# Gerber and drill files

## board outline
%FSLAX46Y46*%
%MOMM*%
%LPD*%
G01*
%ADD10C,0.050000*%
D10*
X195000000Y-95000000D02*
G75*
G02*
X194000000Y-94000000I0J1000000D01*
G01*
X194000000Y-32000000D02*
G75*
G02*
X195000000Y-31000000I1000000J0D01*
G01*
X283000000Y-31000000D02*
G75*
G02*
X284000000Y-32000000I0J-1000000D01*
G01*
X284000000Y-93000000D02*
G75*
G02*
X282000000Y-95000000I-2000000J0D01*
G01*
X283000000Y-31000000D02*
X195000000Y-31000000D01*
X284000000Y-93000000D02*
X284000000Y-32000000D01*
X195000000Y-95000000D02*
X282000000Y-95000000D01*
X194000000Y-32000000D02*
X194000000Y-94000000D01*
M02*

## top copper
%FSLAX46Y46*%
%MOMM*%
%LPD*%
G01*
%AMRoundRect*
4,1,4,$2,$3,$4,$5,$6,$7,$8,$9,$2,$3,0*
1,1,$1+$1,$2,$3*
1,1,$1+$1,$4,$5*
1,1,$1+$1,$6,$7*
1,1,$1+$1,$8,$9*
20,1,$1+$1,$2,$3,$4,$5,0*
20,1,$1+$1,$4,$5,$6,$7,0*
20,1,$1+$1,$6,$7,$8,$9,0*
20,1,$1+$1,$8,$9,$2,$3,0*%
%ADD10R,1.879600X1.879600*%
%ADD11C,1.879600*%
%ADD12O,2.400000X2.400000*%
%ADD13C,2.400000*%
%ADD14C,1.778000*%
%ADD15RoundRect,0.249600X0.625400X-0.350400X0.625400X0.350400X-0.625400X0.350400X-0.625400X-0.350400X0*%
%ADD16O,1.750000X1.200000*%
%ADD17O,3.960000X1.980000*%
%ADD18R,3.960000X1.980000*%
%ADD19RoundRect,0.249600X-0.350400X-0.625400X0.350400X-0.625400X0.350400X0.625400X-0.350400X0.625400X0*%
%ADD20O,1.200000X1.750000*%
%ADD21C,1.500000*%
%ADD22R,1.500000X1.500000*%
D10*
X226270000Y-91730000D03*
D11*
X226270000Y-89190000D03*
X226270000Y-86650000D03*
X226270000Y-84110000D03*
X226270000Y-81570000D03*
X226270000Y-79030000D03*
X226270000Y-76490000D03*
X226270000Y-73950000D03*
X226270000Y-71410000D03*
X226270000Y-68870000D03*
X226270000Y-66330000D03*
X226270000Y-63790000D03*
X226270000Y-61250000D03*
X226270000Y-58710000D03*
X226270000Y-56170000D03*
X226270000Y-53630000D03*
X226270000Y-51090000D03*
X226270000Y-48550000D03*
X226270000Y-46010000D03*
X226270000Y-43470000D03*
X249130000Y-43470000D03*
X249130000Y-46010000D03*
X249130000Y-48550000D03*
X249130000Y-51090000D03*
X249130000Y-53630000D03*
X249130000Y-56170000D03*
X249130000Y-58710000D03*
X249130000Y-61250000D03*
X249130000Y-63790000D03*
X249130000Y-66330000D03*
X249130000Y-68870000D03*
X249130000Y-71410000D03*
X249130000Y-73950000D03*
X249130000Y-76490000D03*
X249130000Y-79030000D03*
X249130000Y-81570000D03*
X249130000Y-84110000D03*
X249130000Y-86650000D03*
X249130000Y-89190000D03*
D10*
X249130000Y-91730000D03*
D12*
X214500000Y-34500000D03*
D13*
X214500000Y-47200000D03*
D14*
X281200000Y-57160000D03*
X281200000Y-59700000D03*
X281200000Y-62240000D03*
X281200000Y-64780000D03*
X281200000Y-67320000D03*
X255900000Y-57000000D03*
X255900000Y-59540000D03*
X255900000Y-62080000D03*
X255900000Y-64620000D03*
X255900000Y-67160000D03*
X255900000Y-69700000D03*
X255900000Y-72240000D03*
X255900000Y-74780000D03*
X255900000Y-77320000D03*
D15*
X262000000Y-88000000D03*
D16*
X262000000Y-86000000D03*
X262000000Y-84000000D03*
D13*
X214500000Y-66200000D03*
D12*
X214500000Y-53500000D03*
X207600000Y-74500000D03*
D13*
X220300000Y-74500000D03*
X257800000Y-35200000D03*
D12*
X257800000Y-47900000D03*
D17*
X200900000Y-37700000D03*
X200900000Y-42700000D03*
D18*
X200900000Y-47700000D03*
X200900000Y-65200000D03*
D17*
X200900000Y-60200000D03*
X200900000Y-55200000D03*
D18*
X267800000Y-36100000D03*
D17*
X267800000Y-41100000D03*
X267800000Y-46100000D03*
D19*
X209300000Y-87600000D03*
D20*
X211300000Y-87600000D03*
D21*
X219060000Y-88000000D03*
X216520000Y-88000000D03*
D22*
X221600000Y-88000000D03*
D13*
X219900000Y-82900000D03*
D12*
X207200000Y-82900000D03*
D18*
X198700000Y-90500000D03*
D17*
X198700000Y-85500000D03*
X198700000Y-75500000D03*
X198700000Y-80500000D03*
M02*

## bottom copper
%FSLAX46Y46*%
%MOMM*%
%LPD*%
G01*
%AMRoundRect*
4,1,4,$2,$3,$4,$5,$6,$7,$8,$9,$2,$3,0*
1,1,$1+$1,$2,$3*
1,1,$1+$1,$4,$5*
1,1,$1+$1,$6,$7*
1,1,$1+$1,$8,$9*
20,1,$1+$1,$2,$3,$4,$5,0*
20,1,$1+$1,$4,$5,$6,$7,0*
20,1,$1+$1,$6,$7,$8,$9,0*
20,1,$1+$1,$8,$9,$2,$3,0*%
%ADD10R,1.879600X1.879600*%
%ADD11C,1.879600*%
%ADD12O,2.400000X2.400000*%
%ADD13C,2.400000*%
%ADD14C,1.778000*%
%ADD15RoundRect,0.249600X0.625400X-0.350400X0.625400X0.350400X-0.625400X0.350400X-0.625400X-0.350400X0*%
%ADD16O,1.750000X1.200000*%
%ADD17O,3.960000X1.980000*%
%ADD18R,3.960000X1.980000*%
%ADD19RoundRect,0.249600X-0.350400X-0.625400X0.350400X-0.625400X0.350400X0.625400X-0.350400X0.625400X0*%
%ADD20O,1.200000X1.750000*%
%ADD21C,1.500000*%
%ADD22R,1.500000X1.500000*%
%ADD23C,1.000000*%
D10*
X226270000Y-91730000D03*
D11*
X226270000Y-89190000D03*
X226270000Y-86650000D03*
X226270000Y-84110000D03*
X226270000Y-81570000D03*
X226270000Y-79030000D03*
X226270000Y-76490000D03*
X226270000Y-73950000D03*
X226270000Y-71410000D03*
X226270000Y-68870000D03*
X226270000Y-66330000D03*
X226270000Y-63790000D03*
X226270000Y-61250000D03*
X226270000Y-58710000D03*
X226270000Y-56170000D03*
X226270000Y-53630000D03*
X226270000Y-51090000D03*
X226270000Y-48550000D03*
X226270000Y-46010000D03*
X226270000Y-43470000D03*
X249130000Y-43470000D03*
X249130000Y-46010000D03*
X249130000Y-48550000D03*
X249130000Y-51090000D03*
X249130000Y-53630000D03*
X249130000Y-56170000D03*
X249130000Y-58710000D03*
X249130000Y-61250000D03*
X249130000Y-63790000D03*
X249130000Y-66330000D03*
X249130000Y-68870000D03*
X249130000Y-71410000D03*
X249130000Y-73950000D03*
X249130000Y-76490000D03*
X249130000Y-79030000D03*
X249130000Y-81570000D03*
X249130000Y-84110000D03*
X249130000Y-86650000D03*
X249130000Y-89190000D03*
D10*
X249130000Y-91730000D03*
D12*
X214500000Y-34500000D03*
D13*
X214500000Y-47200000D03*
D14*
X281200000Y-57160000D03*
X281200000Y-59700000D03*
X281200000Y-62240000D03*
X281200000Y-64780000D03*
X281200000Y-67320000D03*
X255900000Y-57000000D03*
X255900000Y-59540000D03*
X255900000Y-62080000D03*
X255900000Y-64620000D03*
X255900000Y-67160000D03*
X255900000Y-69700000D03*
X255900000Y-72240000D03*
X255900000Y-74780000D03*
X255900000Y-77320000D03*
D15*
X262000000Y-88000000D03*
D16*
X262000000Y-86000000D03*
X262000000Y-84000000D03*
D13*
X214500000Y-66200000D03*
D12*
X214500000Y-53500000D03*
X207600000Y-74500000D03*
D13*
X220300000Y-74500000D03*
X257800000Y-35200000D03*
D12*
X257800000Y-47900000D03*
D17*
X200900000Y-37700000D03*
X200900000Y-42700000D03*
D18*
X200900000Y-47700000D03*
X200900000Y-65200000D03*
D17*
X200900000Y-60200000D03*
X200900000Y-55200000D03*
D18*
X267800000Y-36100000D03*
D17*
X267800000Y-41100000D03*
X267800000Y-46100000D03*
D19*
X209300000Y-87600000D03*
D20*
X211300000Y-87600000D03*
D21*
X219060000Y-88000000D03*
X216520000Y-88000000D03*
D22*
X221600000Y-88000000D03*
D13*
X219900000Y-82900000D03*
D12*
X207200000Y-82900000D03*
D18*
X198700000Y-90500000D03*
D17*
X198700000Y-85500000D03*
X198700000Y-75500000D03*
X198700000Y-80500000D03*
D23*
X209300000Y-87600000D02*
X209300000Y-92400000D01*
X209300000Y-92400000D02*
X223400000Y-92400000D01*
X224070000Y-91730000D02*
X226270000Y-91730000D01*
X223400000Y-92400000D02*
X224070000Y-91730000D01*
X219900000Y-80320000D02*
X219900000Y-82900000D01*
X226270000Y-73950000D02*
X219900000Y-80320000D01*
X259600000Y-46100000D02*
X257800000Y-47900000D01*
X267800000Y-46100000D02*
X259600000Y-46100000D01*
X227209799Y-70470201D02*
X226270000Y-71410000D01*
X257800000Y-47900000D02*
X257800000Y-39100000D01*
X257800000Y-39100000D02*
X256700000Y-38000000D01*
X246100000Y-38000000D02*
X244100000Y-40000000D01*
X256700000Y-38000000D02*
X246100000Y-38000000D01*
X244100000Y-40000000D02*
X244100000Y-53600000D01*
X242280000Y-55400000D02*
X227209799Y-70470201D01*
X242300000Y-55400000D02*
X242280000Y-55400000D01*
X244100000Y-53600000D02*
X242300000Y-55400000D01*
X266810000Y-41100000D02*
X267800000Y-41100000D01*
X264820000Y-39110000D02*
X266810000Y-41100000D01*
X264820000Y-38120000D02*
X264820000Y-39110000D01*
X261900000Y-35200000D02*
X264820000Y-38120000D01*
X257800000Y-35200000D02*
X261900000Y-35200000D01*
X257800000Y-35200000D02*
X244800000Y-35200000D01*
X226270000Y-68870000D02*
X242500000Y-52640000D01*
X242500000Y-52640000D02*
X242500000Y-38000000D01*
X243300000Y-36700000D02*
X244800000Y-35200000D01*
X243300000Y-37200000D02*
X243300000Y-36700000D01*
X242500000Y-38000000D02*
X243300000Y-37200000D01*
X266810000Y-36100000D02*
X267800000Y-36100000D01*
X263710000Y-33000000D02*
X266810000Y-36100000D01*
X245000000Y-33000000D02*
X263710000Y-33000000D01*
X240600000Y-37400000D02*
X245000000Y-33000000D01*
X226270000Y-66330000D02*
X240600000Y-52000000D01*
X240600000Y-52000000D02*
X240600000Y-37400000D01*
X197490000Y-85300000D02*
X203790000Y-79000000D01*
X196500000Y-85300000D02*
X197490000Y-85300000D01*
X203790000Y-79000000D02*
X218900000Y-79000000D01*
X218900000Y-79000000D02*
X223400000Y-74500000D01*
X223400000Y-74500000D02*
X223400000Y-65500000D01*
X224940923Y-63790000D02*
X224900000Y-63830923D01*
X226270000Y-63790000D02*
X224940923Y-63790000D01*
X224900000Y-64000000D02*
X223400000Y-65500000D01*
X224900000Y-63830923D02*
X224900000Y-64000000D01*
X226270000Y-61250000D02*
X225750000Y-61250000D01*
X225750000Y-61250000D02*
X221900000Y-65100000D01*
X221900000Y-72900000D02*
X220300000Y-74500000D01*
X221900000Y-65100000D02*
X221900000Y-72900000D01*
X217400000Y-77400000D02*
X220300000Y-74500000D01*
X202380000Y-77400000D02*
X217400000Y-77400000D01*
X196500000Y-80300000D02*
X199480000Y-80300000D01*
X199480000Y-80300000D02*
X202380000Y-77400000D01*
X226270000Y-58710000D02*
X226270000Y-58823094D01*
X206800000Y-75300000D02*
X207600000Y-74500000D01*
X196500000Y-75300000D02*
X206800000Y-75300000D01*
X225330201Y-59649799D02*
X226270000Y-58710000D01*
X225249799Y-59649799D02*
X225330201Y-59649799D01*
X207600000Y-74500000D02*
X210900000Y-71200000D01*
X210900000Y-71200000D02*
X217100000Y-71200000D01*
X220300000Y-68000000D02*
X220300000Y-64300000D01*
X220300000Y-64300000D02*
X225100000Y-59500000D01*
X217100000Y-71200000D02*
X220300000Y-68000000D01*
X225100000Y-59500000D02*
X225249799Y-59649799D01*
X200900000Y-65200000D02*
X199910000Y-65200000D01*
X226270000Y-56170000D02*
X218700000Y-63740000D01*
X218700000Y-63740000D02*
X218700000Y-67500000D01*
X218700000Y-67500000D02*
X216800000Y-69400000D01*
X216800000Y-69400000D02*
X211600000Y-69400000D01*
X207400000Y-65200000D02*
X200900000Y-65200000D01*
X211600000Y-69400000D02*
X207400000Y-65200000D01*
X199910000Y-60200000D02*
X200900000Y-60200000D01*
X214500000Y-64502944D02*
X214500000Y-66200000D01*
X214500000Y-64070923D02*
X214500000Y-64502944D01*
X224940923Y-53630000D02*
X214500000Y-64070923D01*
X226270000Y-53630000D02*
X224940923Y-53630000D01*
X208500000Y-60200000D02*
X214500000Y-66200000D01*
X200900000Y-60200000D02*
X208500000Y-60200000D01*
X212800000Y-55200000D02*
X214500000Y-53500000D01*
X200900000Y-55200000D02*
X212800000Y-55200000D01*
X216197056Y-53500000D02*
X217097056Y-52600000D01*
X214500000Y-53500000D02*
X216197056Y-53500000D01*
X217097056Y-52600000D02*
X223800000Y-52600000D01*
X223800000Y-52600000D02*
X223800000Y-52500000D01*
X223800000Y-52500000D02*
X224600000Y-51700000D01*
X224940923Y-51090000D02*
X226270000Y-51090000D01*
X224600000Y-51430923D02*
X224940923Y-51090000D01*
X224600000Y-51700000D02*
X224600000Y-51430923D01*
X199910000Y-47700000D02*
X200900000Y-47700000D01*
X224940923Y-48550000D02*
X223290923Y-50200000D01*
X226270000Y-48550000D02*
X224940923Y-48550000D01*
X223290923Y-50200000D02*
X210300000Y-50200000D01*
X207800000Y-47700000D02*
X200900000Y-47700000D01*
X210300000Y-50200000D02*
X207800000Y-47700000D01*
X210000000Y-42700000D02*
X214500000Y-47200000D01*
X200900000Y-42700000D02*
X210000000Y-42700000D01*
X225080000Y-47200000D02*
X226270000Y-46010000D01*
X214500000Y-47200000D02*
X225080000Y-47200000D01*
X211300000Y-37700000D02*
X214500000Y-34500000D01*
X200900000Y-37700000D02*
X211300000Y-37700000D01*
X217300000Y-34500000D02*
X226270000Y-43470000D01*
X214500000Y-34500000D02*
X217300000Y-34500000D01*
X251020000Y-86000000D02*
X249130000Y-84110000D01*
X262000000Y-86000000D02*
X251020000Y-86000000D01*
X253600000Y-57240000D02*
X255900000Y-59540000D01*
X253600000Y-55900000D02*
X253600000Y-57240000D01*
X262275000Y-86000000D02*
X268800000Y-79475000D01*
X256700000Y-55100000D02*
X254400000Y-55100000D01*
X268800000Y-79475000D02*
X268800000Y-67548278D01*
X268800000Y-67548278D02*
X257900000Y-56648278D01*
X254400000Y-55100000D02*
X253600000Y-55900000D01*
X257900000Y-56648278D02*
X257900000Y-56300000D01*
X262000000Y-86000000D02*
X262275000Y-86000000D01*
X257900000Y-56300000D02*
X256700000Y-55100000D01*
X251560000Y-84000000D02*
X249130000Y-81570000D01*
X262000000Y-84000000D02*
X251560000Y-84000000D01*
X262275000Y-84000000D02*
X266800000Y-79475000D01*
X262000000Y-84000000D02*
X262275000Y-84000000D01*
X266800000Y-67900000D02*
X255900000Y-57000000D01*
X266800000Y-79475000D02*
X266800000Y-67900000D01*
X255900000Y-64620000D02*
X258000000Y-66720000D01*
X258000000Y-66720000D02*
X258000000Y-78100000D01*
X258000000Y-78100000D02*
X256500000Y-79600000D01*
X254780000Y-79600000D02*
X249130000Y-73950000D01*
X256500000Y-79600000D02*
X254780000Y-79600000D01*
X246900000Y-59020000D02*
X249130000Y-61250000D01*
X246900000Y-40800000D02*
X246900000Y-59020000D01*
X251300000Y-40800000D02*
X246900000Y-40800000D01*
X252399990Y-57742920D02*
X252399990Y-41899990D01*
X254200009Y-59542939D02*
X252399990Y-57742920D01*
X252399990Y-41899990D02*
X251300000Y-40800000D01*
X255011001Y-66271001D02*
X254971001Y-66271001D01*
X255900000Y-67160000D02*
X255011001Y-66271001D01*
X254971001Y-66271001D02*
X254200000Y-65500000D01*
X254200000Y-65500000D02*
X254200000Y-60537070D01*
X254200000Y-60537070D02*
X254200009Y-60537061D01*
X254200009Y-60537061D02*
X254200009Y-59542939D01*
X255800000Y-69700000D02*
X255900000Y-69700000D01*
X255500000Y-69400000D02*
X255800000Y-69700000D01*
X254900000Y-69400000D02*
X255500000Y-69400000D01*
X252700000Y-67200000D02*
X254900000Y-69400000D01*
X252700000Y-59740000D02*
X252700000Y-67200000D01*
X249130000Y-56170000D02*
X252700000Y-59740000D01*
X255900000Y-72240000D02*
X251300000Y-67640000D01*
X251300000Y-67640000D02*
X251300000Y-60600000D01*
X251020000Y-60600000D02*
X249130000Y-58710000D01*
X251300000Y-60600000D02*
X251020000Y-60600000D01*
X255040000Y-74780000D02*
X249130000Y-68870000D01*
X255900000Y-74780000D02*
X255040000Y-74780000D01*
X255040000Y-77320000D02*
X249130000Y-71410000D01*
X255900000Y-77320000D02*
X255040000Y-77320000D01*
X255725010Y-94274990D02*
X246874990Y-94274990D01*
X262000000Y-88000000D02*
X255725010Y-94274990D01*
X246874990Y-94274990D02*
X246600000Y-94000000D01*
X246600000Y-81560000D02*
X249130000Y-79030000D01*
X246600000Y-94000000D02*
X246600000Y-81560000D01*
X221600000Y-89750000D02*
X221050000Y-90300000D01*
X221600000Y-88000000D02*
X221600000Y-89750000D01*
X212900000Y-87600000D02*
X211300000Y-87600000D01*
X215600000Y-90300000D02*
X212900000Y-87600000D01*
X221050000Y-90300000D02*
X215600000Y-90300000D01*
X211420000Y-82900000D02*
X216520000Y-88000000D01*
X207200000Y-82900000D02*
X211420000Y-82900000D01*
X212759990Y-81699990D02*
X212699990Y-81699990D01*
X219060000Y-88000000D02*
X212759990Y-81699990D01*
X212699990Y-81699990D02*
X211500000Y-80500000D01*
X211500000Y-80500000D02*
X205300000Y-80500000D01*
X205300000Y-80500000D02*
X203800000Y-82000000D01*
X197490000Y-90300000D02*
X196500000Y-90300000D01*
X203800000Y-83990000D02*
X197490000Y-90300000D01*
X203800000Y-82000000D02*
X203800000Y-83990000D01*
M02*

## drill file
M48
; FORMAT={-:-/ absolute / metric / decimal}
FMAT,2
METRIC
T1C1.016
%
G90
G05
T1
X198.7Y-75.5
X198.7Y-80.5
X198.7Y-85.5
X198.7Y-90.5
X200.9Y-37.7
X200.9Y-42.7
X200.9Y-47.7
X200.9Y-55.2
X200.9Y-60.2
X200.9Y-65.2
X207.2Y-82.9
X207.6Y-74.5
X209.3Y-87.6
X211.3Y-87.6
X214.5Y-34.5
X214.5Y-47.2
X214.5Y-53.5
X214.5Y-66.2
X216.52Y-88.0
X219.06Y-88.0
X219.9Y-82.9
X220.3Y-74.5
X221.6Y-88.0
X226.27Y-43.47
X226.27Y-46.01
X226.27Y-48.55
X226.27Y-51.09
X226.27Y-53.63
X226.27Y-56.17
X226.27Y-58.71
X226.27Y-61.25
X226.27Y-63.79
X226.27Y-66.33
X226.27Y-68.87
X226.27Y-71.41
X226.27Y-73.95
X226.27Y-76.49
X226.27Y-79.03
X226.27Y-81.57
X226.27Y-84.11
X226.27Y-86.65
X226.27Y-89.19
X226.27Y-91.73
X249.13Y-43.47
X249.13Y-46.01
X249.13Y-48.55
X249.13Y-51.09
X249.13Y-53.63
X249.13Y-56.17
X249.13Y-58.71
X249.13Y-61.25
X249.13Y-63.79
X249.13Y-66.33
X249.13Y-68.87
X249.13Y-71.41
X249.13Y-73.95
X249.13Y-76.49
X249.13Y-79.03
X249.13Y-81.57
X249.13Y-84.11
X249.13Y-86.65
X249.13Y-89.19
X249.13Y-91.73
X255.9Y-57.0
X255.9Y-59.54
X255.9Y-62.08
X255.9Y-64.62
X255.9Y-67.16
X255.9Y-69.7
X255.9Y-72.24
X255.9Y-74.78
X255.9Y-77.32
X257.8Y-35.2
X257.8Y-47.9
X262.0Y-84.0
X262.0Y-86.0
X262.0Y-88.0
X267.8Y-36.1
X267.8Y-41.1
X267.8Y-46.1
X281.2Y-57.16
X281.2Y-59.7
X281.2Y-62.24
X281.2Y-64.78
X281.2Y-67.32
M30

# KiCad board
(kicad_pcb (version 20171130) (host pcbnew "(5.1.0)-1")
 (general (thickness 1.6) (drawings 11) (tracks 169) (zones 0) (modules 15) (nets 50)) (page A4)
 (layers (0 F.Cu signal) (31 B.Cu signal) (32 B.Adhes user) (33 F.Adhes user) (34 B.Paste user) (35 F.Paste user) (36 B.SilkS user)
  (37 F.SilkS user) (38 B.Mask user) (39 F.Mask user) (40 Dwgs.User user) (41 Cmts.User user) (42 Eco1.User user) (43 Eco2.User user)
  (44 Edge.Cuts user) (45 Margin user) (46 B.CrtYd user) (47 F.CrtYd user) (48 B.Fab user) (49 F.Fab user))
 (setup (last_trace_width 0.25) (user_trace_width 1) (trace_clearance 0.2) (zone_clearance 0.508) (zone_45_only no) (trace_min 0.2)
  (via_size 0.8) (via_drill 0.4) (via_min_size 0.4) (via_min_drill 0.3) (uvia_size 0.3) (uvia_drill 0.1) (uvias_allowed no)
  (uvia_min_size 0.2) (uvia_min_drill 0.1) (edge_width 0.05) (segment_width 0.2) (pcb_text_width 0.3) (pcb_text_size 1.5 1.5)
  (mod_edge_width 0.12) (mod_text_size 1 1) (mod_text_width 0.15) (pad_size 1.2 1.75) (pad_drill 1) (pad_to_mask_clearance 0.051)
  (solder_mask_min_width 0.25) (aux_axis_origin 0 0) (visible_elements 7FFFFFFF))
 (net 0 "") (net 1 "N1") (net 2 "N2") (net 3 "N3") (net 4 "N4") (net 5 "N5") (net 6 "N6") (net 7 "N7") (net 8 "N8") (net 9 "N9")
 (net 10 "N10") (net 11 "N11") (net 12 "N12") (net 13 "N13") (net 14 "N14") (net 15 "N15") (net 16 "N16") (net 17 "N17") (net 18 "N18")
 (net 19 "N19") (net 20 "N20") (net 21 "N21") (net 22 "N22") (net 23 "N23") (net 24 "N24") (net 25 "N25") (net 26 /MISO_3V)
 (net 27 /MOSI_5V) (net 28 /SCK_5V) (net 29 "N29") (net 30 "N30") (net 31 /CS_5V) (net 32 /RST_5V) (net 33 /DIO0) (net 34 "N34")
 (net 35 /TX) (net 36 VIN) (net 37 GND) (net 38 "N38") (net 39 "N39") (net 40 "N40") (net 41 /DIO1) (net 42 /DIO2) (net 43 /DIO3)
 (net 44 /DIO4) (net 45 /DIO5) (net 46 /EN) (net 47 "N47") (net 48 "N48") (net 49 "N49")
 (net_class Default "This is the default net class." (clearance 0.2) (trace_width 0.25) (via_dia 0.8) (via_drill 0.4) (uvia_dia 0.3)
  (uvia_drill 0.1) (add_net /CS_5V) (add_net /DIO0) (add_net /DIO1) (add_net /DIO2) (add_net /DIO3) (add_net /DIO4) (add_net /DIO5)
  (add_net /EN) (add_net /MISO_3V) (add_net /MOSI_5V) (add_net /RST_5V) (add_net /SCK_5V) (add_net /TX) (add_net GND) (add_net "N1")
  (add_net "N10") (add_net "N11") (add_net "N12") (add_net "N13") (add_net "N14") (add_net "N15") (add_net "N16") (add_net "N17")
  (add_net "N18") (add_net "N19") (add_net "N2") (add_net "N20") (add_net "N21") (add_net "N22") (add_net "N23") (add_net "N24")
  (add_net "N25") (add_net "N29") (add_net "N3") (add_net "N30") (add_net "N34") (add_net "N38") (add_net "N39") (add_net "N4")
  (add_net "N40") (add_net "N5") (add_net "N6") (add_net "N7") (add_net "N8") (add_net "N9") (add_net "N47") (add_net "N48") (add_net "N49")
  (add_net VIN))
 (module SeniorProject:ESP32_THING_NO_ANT (layer F.Cu) (at 225 93)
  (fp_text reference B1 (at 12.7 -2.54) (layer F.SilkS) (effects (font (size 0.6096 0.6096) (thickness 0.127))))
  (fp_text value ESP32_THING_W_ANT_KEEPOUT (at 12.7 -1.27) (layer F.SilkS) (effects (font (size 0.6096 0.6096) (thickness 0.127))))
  (pad 1 thru_hole rect (at 1.27 -1.27) (size 1.8796 1.8796) (drill 1.016) (layers *.Cu *.Mask) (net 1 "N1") (solder_mask_margin 0.1016))
  (pad 2 thru_hole circle (at 1.27 -3.81) (size 1.8796 1.8796) (drill 1.016) (layers *.Cu *.Mask) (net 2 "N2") (solder_mask_margin 0.1016))
  (pad 3 thru_hole circle (at 1.27 -6.35) (size 1.8796 1.8796) (drill 1.016) (layers *.Cu *.Mask) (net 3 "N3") (solder_mask_margin 0.1016))
  (pad 4 thru_hole circle (at 1.27 -8.89) (size 1.8796 1.8796) (drill 1.016) (layers *.Cu *.Mask) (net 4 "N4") (solder_mask_margin 0.1016))
  (pad 5 thru_hole circle (at 1.27 -11.43) (size 1.8796 1.8796) (drill 1.016) (layers *.Cu *.Mask) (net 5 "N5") (solder_mask_margin 0.1016))
  (pad 6 thru_hole circle (at 1.27 -13.97) (size 1.8796 1.8796) (drill 1.016) (layers *.Cu *.Mask) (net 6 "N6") (solder_mask_margin 0.1016))
  (pad 7 thru_hole circle (at 1.27 -16.51) (size 1.8796 1.8796) (drill 1.016) (layers *.Cu *.Mask) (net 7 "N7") (solder_mask_margin 0.1016))
  (pad 8 thru_hole circle (at 1.27 -19.05) (size 1.8796 1.8796) (drill 1.016) (layers *.Cu *.Mask) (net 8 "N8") (solder_mask_margin 0.1016))
  (pad 9 thru_hole circle (at 1.27 -21.59) (size 1.8796 1.8796) (drill 1.016) (layers *.Cu *.Mask) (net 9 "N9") (solder_mask_margin 0.1016))
  (pad 10 thru_hole circle (at 1.27 -24.13) (size 1.8796 1.8796) (drill 1.016) (layers *.Cu *.Mask) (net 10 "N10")
   (solder_mask_margin 0.1016))
  (pad 11 thru_hole circle (at 1.27 -26.67) (size 1.8796 1.8796) (drill 1.016) (layers *.Cu *.Mask) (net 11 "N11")
   (solder_mask_margin 0.1016))
  (pad 12 thru_hole circle (at 1.27 -29.21) (size 1.8796 1.8796) (drill 1.016) (layers *.Cu *.Mask) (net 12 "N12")
   (solder_mask_margin 0.1016))
  (pad 13 thru_hole circle (at 1.27 -31.75) (size 1.8796 1.8796) (drill 1.016) (layers *.Cu *.Mask) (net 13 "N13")
   (solder_mask_margin 0.1016))
  (pad 14 thru_hole circle (at 1.27 -34.29) (size 1.8796 1.8796) (drill 1.016) (layers *.Cu *.Mask) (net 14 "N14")
   (solder_mask_margin 0.1016))
  (pad 15 thru_hole circle (at 1.27 -36.83) (size 1.8796 1.8796) (drill 1.016) (layers *.Cu *.Mask) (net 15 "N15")
   (solder_mask_margin 0.1016))
  (pad 16 thru_hole circle (at 1.27 -39.37) (size 1.8796 1.8796) (drill 1.016) (layers *.Cu *.Mask) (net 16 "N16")
   (solder_mask_margin 0.1016))
  (pad 17 thru_hole circle (at 1.27 -41.91) (size 1.8796 1.8796) (drill 1.016) (layers *.Cu *.Mask) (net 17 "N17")
   (solder_mask_margin 0.1016))
  (pad 18 thru_hole circle (at 1.27 -44.45) (size 1.8796 1.8796) (drill 1.016) (layers *.Cu *.Mask) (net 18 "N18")
   (solder_mask_margin 0.1016))
  (pad 19 thru_hole circle (at 1.27 -46.99) (size 1.8796 1.8796) (drill 1.016) (layers *.Cu *.Mask) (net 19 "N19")
   (solder_mask_margin 0.1016))
  (pad 20 thru_hole circle (at 1.27 -49.53) (size 1.8796 1.8796) (drill 1.016) (layers *.Cu *.Mask) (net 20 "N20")
   (solder_mask_margin 0.1016))
  (pad 21 thru_hole circle (at 24.13 -49.53) (size 1.8796 1.8796) (drill 1.016) (layers *.Cu *.Mask) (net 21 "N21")
   (solder_mask_margin 0.1016))
  (pad 22 thru_hole circle (at 24.13 -46.99) (size 1.8796 1.8796) (drill 1.016) (layers *.Cu *.Mask) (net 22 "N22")
   (solder_mask_margin 0.1016))
  (pad 23 thru_hole circle (at 24.13 -44.45) (size 1.8796 1.8796) (drill 1.016) (layers *.Cu *.Mask) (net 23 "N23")
   (solder_mask_margin 0.1016))
  (pad 24 thru_hole circle (at 24.13 -41.91) (size 1.8796 1.8796) (drill 1.016) (layers *.Cu *.Mask) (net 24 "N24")
   (solder_mask_margin 0.1016))
  (pad 25 thru_hole circle (at 24.13 -39.37) (size 1.8796 1.8796) (drill 1.016) (layers *.Cu *.Mask) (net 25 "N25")
   (solder_mask_margin 0.1016))
  (pad 26 thru_hole circle (at 24.13 -36.83) (size 1.8796 1.8796) (drill 1.016) (layers *.Cu *.Mask) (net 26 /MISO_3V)
   (solder_mask_margin 0.1016))
  (pad 27 thru_hole circle (at 24.13 -34.29) (size 1.8796 1.8796) (drill 1.016) (layers *.Cu *.Mask) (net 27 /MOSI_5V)
   (solder_mask_margin 0.1016))
  (pad 28 thru_hole circle (at 24.13 -31.75) (size 1.8796 1.8796) (drill 1.016) (layers *.Cu *.Mask) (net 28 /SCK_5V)
   (solder_mask_margin 0.1016))
  (pad 29 thru_hole circle (at 24.13 -29.21) (size 1.8796 1.8796) (drill 1.016) (layers *.Cu *.Mask) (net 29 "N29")
   (solder_mask_margin 0.1016))
  (pad 30 thru_hole circle (at 24.13 -26.67) (size 1.8796 1.8796) (drill 1.016) (layers *.Cu *.Mask) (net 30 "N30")
   (solder_mask_margin 0.1016))
  (pad 31 thru_hole circle (at 24.13 -24.13) (size 1.8796 1.8796) (drill 1.016) (layers *.Cu *.Mask) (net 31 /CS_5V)
   (solder_mask_margin 0.1016))
  (pad 32 thru_hole circle (at 24.13 -21.59) (size 1.8796 1.8796) (drill 1.016) (layers *.Cu *.Mask) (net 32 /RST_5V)
   (solder_mask_margin 0.1016))
  (pad 33 thru_hole circle (at 24.13 -19.05) (size 1.8796 1.8796) (drill 1.016) (layers *.Cu *.Mask) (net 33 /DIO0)
   (solder_mask_margin 0.1016))
  (pad 34 thru_hole circle (at 24.13 -16.51) (size 1.8796 1.8796) (drill 1.016) (layers *.Cu *.Mask) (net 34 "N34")
   (solder_mask_margin 0.1016))
  (pad 35 thru_hole circle (at 24.13 -13.97) (size 1.8796 1.8796) (drill 1.016) (layers *.Cu *.Mask) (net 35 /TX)
   (solder_mask_margin 0.1016))
  (pad 36 thru_hole circle (at 24.13 -11.43) (size 1.8796 1.8796) (drill 1.016) (layers *.Cu *.Mask) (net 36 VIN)
   (solder_mask_margin 0.1016))
  (pad 37 thru_hole circle (at 24.13 -8.89) (size 1.8796 1.8796) (drill 1.016) (layers *.Cu *.Mask) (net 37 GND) (solder_mask_margin 0.1016))
  (pad 38 thru_hole circle (at 24.13 -6.35) (size 1.8796 1.8796) (drill 1.016) (layers *.Cu *.Mask) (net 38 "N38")
   (solder_mask_margin 0.1016))
  (pad 39 thru_hole circle (at 24.13 -3.81) (size 1.8796 1.8796) (drill 1.016) (layers *.Cu *.Mask) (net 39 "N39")
   (solder_mask_margin 0.1016))
  (pad 40 thru_hole rect (at 24.13 -1.27) (size 1.8796 1.8796) (drill 1.016) (layers *.Cu *.Mask) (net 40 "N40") (solder_mask_margin 0.1016)))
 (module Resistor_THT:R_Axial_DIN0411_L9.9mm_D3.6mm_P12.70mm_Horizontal (layer F.Cu) (at 214.5 47.2 90)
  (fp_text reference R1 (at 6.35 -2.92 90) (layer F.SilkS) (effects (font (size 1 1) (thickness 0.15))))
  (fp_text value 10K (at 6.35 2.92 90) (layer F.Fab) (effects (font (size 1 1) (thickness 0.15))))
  (pad 2 thru_hole oval (at 12.7 0 90) (size 2.4 2.4) (drill 1.016) (layers *.Cu *.Mask) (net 20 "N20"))
  (pad 1 thru_hole circle (at 0 0 90) (size 2.4 2.4) (drill 1.016) (layers *.Cu *.Mask) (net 19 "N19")))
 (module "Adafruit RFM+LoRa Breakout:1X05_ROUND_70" (layer F.Cu) (at 281.2 62.24 270)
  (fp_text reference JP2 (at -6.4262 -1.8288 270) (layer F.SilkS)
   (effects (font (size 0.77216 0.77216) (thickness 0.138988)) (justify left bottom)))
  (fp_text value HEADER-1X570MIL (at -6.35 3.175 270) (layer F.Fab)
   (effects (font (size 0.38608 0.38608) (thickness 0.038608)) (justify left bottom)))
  (pad 1 thru_hole circle (at -5.08 0) (size 1.778 1.778) (drill 1.016) (layers *.Cu *.Mask) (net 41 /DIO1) (solder_mask_margin 0.0508))
  (pad 2 thru_hole circle (at -2.54 0) (size 1.778 1.778) (drill 1.016) (layers *.Cu *.Mask) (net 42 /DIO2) (solder_mask_margin 0.0508))
  (pad 3 thru_hole circle (at 0 0) (size 1.778 1.778) (drill 1.016) (layers *.Cu *.Mask) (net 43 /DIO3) (solder_mask_margin 0.0508))
  (pad 4 thru_hole circle (at 2.54 0) (size 1.778 1.778) (drill 1.016) (layers *.Cu *.Mask) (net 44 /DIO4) (solder_mask_margin 0.0508))
  (pad 5 thru_hole circle (at 5.08 0) (size 1.778 1.778) (drill 1.016) (layers *.Cu *.Mask) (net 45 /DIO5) (solder_mask_margin 0.0508)))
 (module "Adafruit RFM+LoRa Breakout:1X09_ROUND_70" (layer F.Cu) (at 255.9 67.16 270)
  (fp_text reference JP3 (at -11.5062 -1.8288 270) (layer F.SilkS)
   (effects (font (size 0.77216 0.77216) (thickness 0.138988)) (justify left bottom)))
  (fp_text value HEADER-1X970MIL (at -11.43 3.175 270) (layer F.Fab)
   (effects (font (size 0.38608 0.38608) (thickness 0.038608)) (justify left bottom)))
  (pad 1 thru_hole circle (at -10.16 0) (size 1.778 1.778) (drill 1.016) (layers *.Cu *.Mask) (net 36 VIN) (solder_mask_margin 0.0508))
  (pad 2 thru_hole circle (at -7.62 0) (size 1.778 1.778) (drill 1.016) (layers *.Cu *.Mask) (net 37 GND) (solder_mask_margin 0.0508))
  (pad 3 thru_hole circle (at -5.08 0) (size 1.778 1.778) (drill 1.016) (layers *.Cu *.Mask) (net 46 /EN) (solder_mask_margin 0.0508))
  (pad 4 thru_hole circle (at -2.54 0) (size 1.778 1.778) (drill 1.016) (layers *.Cu *.Mask) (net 33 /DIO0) (solder_mask_margin 0.0508))
  (pad 5 thru_hole circle (at 0 0) (size 1.778 1.778) (drill 1.016) (layers *.Cu *.Mask) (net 28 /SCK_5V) (solder_mask_margin 0.0508))
  (pad 6 thru_hole circle (at 2.54 0) (size 1.778 1.778) (drill 1.016) (layers *.Cu *.Mask) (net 26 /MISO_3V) (solder_mask_margin 0.0508))
  (pad 7 thru_hole circle (at 5.08 0) (size 1.778 1.778) (drill 1.016) (layers *.Cu *.Mask) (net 27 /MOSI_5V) (solder_mask_margin 0.0508))
  (pad 8 thru_hole circle (at 7.62 0) (size 1.778 1.778) (drill 1.016) (layers *.Cu *.Mask) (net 31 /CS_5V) (solder_mask_margin 0.0508))
  (pad 9 thru_hole circle (at 10.16 0) (size 1.778 1.778) (drill 1.016) (layers *.Cu *.Mask) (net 32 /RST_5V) (solder_mask_margin 0.0508)))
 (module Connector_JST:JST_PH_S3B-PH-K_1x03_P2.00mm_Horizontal (layer F.Cu) (at 262 88 90)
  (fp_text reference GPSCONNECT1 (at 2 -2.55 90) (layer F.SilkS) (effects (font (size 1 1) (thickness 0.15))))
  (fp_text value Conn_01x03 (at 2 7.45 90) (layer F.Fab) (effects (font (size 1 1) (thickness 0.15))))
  (pad 1 thru_hole roundrect (at 0 0 90) (size 1.2 1.75) (drill 1.016) (layers *.Cu *.Mask) (roundrect_rratio 0.208) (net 35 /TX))
  (pad 2 thru_hole oval (at 2 0 90) (size 1.2 1.75) (drill 1.016) (layers *.Cu *.Mask) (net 37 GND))
  (pad 3 thru_hole oval (at 4 0 90) (size 1.2 1.75) (drill 1.016) (layers *.Cu *.Mask) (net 36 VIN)))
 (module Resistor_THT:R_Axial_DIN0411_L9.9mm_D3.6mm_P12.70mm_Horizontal (layer F.Cu) (at 214.5 66.2 90)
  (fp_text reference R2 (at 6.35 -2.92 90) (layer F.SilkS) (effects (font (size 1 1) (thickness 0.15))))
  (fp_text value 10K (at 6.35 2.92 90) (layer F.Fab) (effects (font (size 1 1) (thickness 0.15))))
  (pad 1 thru_hole circle (at 0 0 90) (size 2.4 2.4) (drill 1.016) (layers *.Cu *.Mask) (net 16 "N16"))
  (pad 2 thru_hole oval (at 12.7 0 90) (size 2.4 2.4) (drill 1.016) (layers *.Cu *.Mask) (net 17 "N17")))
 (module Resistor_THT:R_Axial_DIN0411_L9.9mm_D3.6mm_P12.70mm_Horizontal (layer F.Cu) (at 220.3 74.5 180)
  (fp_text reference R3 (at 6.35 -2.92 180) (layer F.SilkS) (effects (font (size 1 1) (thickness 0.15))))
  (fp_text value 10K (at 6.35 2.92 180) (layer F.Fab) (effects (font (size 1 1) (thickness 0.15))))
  (pad 2 thru_hole oval (at 12.7 0 180) (size 2.4 2.4) (drill 1.016) (layers *.Cu *.Mask) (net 14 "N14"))
  (pad 1 thru_hole circle (at 0 0 180) (size 2.4 2.4) (drill 1.016) (layers *.Cu *.Mask) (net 13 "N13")))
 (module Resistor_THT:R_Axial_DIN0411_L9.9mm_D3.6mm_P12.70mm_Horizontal (layer F.Cu) (at 257.8 35.2 270)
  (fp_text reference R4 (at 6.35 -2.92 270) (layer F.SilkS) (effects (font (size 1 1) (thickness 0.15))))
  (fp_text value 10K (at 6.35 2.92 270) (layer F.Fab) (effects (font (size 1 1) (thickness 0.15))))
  (pad 1 thru_hole circle (at 0 0 270) (size 2.4 2.4) (drill 1.016) (layers *.Cu *.Mask) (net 10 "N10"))
  (pad 2 thru_hole oval (at 12.7 0 270) (size 2.4 2.4) (drill 1.016) (layers *.Cu *.Mask) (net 9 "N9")))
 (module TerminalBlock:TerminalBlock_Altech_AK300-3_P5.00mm (layer F.Cu) (at 200.9 47.7 90)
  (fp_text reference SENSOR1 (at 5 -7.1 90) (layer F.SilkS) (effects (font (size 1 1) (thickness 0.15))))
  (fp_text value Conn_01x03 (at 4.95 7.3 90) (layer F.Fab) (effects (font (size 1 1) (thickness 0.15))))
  (pad 3 thru_hole oval (at 10 0 90) (size 1.98 3.96) (drill 1.016) (layers *.Cu *.Mask) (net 20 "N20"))
  (pad 2 thru_hole oval (at 5 0 90) (size 1.98 3.96) (drill 1.016) (layers *.Cu *.Mask) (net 19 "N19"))
  (pad 1 thru_hole rect (at 0 0 90) (size 1.98 3.96) (drill 1.016) (layers *.Cu *.Mask) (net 18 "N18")))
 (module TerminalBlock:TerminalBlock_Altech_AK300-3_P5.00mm (layer F.Cu) (at 200.9 65.2 90)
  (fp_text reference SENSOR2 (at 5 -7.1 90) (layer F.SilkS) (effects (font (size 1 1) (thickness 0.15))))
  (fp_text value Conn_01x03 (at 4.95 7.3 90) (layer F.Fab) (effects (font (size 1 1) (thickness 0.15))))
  (pad 1 thru_hole rect (at 0 0 90) (size 1.98 3.96) (drill 1.016) (layers *.Cu *.Mask) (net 15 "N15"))
  (pad 2 thru_hole oval (at 5 0 90) (size 1.98 3.96) (drill 1.016) (layers *.Cu *.Mask) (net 16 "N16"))
  (pad 3 thru_hole oval (at 10 0 90) (size 1.98 3.96) (drill 1.016) (layers *.Cu *.Mask) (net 17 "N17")))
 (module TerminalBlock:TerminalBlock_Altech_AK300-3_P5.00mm (layer F.Cu) (at 267.8 36.1 270)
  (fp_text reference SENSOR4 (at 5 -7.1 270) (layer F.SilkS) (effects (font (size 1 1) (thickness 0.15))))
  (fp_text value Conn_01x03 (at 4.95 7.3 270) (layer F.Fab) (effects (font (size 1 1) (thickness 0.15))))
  (pad 1 thru_hole rect (at 0 0 270) (size 1.98 3.96) (drill 1.016) (layers *.Cu *.Mask) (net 11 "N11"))
  (pad 2 thru_hole oval (at 5 0 270) (size 1.98 3.96) (drill 1.016) (layers *.Cu *.Mask) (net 10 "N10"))
  (pad 3 thru_hole oval (at 10 0 270) (size 1.98 3.96) (drill 1.016) (layers *.Cu *.Mask) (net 9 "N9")))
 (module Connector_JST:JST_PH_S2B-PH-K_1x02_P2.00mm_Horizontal (layer F.Cu) (at 209.3 87.6)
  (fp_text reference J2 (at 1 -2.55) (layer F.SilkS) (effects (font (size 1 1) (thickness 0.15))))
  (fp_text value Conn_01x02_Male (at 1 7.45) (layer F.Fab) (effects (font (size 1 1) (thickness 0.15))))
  (pad 1 thru_hole roundrect (at 0 0) (size 1.2 1.75) (drill 1.016) (layers *.Cu *.Mask) (roundrect_rratio 0.208) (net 1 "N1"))
  (pad 2 thru_hole oval (at 2 0) (size 1.2 1.75) (drill 1.016) (layers *.Cu *.Mask) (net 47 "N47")))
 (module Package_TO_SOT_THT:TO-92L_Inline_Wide (layer F.Cu) (at 221.6 88 180)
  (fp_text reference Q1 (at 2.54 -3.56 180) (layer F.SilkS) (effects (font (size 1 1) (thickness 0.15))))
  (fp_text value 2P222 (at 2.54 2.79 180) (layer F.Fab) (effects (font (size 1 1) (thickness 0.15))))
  (pad 2 thru_hole circle (at 2.54 0 270) (size 1.5 1.5) (drill 1.016) (layers *.Cu *.Mask) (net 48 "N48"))
  (pad 3 thru_hole circle (at 5.08 0 270) (size 1.5 1.5) (drill 1.016) (layers *.Cu *.Mask) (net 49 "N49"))
  (pad 1 thru_hole rect (at 0 0 270) (size 1.5 1.5) (drill 1.016) (layers *.Cu *.Mask) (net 47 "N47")))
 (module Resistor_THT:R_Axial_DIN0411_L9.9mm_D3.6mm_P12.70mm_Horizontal (layer F.Cu) (at 219.9 82.9 180)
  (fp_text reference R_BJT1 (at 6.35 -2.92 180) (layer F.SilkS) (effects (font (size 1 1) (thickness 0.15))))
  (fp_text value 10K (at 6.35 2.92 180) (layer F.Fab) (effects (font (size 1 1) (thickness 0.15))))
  (pad 1 thru_hole circle (at 0 0 180) (size 2.4 2.4) (drill 1.016) (layers *.Cu *.Mask) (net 8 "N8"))
  (pad 2 thru_hole oval (at 12.7 0 180) (size 2.4 2.4) (drill 1.016) (layers *.Cu *.Mask) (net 49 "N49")))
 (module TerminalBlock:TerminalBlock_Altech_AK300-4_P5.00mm (layer F.Cu) (at 198.7 90.5 90)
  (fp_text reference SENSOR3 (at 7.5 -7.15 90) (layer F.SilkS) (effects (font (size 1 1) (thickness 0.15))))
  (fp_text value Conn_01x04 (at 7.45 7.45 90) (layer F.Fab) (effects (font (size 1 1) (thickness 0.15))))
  (pad 1 thru_hole rect (at 0 0 90) (size 1.98 3.96) (drill 1.016) (layers *.Cu *.Mask) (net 48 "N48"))
  (pad 2 thru_hole oval (at 5 0 90) (size 1.98 3.96) (drill 1.016) (layers *.Cu *.Mask) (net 12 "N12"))
  (pad 4 thru_hole oval (at 15 0 90) (size 1.98 3.96) (drill 1.016) (layers *.Cu *.Mask) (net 14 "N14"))
  (pad 3 thru_hole oval (at 10 0 90) (size 1.98 3.96) (drill 1.016) (layers *.Cu *.Mask) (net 13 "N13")))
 (gr_arc (start 195 94) (end 194 94) (angle -90) (layer Edge.Cuts) (width 0.05))
 (gr_arc (start 195 32) (end 195 31) (angle -90) (layer Edge.Cuts) (width 0.05))
 (gr_arc (start 283 32) (end 284 32) (angle -90) (layer Edge.Cuts) (width 0.05))
 (gr_arc (start 282 93) (end 282 95) (angle -90) (layer Edge.Cuts) (width 0.05))
 (gr_line (start 283 31) (end 195 31) (layer Edge.Cuts) (width 0.05))
 (gr_line (start 284 93) (end 284 32) (layer Edge.Cuts) (width 0.05))
 (gr_line (start 195 95) (end 282 95) (layer Edge.Cuts) (width 0.05))
 (gr_line (start 194 32) (end 194 94) (layer Edge.Cuts) (width 0.05))
 (segment (start 209.3 87.6) (end 209.3 92.4) (width 1) (layer B.Cu) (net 1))
 (segment (start 209.3 92.4) (end 223.4 92.4) (width 1) (layer B.Cu) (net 1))
 (segment (start 224.07 91.73) (end 226.27 91.73) (width 1) (layer B.Cu) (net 1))
 (segment (start 223.4 92.4) (end 224.07 91.73) (width 1) (layer B.Cu) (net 1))
 (segment (start 219.9 80.32) (end 219.9 82.9) (width 1) (layer B.Cu) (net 8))
 (segment (start 226.27 73.95) (end 219.9 80.32) (width 1) (layer B.Cu) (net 8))
 (segment (start 259.6 46.1) (end 257.8 47.9) (width 1) (layer B.Cu) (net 9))
 (segment (start 267.8 46.1) (end 259.6 46.1) (width 1) (layer B.Cu) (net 9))
 (segment (start 227.209799 70.470201) (end 226.27 71.41) (width 1) (layer B.Cu) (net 9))
 (segment (start 257.8 47.9) (end 257.8 39.1) (width 1) (layer B.Cu) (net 9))
 (segment (start 257.8 39.1) (end 256.7 38) (width 1) (layer B.Cu) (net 9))
 (segment (start 246.1 38) (end 244.1 40) (width 1) (layer B.Cu) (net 9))
 (segment (start 256.7 38) (end 246.1 38) (width 1) (layer B.Cu) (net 9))
 (segment (start 244.1 40) (end 244.1 53.6) (width 1) (layer B.Cu) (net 9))
 (segment (start 242.28 55.4) (end 227.209799 70.470201) (width 1) (layer B.Cu) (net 9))
 (segment (start 242.3 55.4) (end 242.28 55.4) (width 1) (layer B.Cu) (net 9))
 (segment (start 244.1 53.6) (end 242.3 55.4) (width 1) (layer B.Cu) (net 9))
 (segment (start 266.81 41.1) (end 267.8 41.1) (width 1) (layer B.Cu) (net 10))
 (segment (start 264.82 39.11) (end 266.81 41.1) (width 1) (layer B.Cu) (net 10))
 (segment (start 264.82 38.12) (end 264.82 39.11) (width 1) (layer B.Cu) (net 10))
 (segment (start 261.9 35.2) (end 264.82 38.12) (width 1) (layer B.Cu) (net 10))
 (segment (start 257.8 35.2) (end 261.9 35.2) (width 1) (layer B.Cu) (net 10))
 (segment (start 257.8 35.2) (end 244.8 35.2) (width 1) (layer B.Cu) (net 10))
 (segment (start 226.27 68.87) (end 242.5 52.64) (width 1) (layer B.Cu) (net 10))
 (segment (start 242.5 52.64) (end 242.5 38) (width 1) (layer B.Cu) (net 10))
 (segment (start 243.3 36.7) (end 244.8 35.2) (width 1) (layer B.Cu) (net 10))
 (segment (start 243.3 37.2) (end 243.3 36.7) (width 1) (layer B.Cu) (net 10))
 (segment (start 242.5 38) (end 243.3 37.2) (width 1) (layer B.Cu) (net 10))
 (segment (start 266.81 36.1) (end 267.8 36.1) (width 1) (layer B.Cu) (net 11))
 (segment (start 263.71 33) (end 266.81 36.1) (width 1) (layer B.Cu) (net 11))
 (segment (start 245 33) (end 263.71 33) (width 1) (layer B.Cu) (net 11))
 (segment (start 240.6 37.4) (end 245 33) (width 1) (layer B.Cu) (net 11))
 (segment (start 226.27 66.33) (end 240.6 52) (width 1) (layer B.Cu) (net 11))
 (segment (start 240.6 52) (end 240.6 37.4) (width 1) (layer B.Cu) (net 11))
 (segment (start 197.49 85.3) (end 203.79 79) (width 1) (layer B.Cu) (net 12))
 (segment (start 196.5 85.3) (end 197.49 85.3) (width 1) (layer B.Cu) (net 12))
 (segment (start 203.79 79) (end 218.9 79) (width 1) (layer B.Cu) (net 12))
 (segment (start 218.9 79) (end 223.4 74.5) (width 1) (layer B.Cu) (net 12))
 (segment (start 223.4 74.5) (end 223.4 65.5) (width 1) (layer B.Cu) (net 12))
 (segment (start 224.940923 63.79) (end 224.9 63.830923) (width 1) (layer B.Cu) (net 12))
 (segment (start 226.27 63.79) (end 224.940923 63.79) (width 1) (layer B.Cu) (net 12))
 (segment (start 224.9 64) (end 223.4 65.5) (width 1) (layer B.Cu) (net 12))
 (segment (start 224.9 63.830923) (end 224.9 64) (width 1) (layer B.Cu) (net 12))
 (segment (start 226.27 61.25) (end 225.75 61.25) (width 1) (layer B.Cu) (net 13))
 (segment (start 225.75 61.25) (end 221.9 65.1) (width 1) (layer B.Cu) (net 13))
 (segment (start 221.9 72.9) (end 220.3 74.5) (width 1) (layer B.Cu) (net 13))
 (segment (start 221.9 65.1) (end 221.9 72.9) (width 1) (layer B.Cu) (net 13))
 (segment (start 217.4 77.4) (end 220.3 74.5) (width 1) (layer B.Cu) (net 13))
 (segment (start 202.38 77.4) (end 217.4 77.4) (width 1) (layer B.Cu) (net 13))
 (segment (start 196.5 80.3) (end 199.48 80.3) (width 1) (layer B.Cu) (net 13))
 (segment (start 199.48 80.3) (end 202.38 77.4) (width 1) (layer B.Cu) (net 13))
 (segment (start 226.27 58.71) (end 226.27 58.823094) (width 1) (layer B.Cu) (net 14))
 (segment (start 206.8 75.3) (end 207.6 74.5) (width 1) (layer B.Cu) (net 14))
 (segment (start 196.5 75.3) (end 206.8 75.3) (width 1) (layer B.Cu) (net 14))
 (segment (start 225.330201 59.649799) (end 226.27 58.71) (width 1) (layer B.Cu) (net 14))
 (segment (start 225.249799 59.649799) (end 225.330201 59.649799) (width 1) (layer B.Cu) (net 14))
 (segment (start 207.6 74.5) (end 210.9 71.2) (width 1) (layer B.Cu) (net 14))
 (segment (start 210.9 71.2) (end 217.1 71.2) (width 1) (layer B.Cu) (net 14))
 (segment (start 220.3 68) (end 220.3 64.3) (width 1) (layer B.Cu) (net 14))
 (segment (start 220.3 64.3) (end 225.1 59.5) (width 1) (layer B.Cu) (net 14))
 (segment (start 217.1 71.2) (end 220.3 68) (width 1) (layer B.Cu) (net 14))
 (segment (start 225.1 59.5) (end 225.249799 59.649799) (width 1) (layer B.Cu) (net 14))
 (segment (start 200.9 65.2) (end 199.91 65.2) (width 1) (layer B.Cu) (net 15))
 (segment (start 226.27 56.17) (end 218.7 63.74) (width 1) (layer B.Cu) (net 15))
 (segment (start 218.7 63.74) (end 218.7 67.5) (width 1) (layer B.Cu) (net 15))
 (segment (start 218.7 67.5) (end 216.8 69.4) (width 1) (layer B.Cu) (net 15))
 (segment (start 216.8 69.4) (end 211.6 69.4) (width 1) (layer B.Cu) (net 15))
 (segment (start 207.4 65.2) (end 200.9 65.2) (width 1) (layer B.Cu) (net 15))
 (segment (start 211.6 69.4) (end 207.4 65.2) (width 1) (layer B.Cu) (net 15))
 (segment (start 199.91 60.2) (end 200.9 60.2) (width 1) (layer B.Cu) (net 16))
 (segment (start 214.5 64.502944) (end 214.5 66.2) (width 1) (layer B.Cu) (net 16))
 (segment (start 214.5 64.070923) (end 214.5 64.502944) (width 1) (layer B.Cu) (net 16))
 (segment (start 224.940923 53.63) (end 214.5 64.070923) (width 1) (layer B.Cu) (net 16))
 (segment (start 226.27 53.63) (end 224.940923 53.63) (width 1) (layer B.Cu) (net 16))
 (segment (start 208.5 60.2) (end 214.5 66.2) (width 1) (layer B.Cu) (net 16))
 (segment (start 200.9 60.2) (end 208.5 60.2) (width 1) (layer B.Cu) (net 16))
 (segment (start 212.8 55.2) (end 214.5 53.5) (width 1) (layer B.Cu) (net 17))
 (segment (start 200.9 55.2) (end 212.8 55.2) (width 1) (layer B.Cu) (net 17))
 (segment (start 216.197056 53.5) (end 217.097056 52.6) (width 1) (layer B.Cu) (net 17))
 (segment (start 214.5 53.5) (end 216.197056 53.5) (width 1) (layer B.Cu) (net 17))
 (segment (start 217.097056 52.6) (end 223.8 52.6) (width 1) (layer B.Cu) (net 17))
 (segment (start 223.8 52.6) (end 223.8 52.5) (width 1) (layer B.Cu) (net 17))
 (segment (start 223.8 52.5) (end 224.6 51.7) (width 1) (layer B.Cu) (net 17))
 (segment (start 224.940923 51.09) (end 226.27 51.09) (width 1) (layer B.Cu) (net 17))
 (segment (start 224.6 51.430923) (end 224.940923 51.09) (width 1) (layer B.Cu) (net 17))
 (segment (start 224.6 51.7) (end 224.6 51.430923) (width 1) (layer B.Cu) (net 17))
 (segment (start 199.91 47.7) (end 200.9 47.7) (width 1) (layer B.Cu) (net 18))
 (segment (start 224.940923 48.55) (end 223.290923 50.2) (width 1) (layer B.Cu) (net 18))
 (segment (start 226.27 48.55) (end 224.940923 48.55) (width 1) (layer B.Cu) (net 18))
 (segment (start 223.290923 50.2) (end 210.3 50.2) (width 1) (layer B.Cu) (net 18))
 (segment (start 207.8 47.7) (end 200.9 47.7) (width 1) (layer B.Cu) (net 18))
 (segment (start 210.3 50.2) (end 207.8 47.7) (width 1) (layer B.Cu) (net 18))
 (segment (start 210 42.7) (end 214.5 47.2) (width 1) (layer B.Cu) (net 19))
 (segment (start 200.9 42.7) (end 210 42.7) (width 1) (layer B.Cu) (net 19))
 (segment (start 225.08 47.2) (end 226.27 46.01) (width 1) (layer B.Cu) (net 19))
 (segment (start 214.5 47.2) (end 225.08 47.2) (width 1) (layer B.Cu) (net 19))
 (segment (start 211.3 37.7) (end 214.5 34.5) (width 1) (layer B.Cu) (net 20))
 (segment (start 200.9 37.7) (end 211.3 37.7) (width 1) (layer B.Cu) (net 20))
 (segment (start 217.3 34.5) (end 226.27 43.47) (width 1) (layer B.Cu) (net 20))
 (segment (start 214.5 34.5) (end 217.3 34.5) (width 1) (layer B.Cu) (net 20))
 (segment (start 251.02 86) (end 249.13 84.11) (width 1) (layer B.Cu) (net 37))
 (segment (start 262 86) (end 251.02 86) (width 1) (layer B.Cu) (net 37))
 (segment (start 253.6 57.24) (end 255.9 59.54) (width 1) (layer B.Cu) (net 37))
 (segment (start 253.6 55.9) (end 253.6 57.24) (width 1) (layer B.Cu) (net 37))
 (segment (start 262.275 86) (end 268.8 79.475) (width 1) (layer B.Cu) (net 37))
 (segment (start 256.7 55.1) (end 254.4 55.1) (width 1) (layer B.Cu) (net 37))
 (segment (start 268.8 79.475) (end 268.8 67.548278) (width 1) (layer B.Cu) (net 37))
 (segment (start 268.8 67.548278) (end 257.9 56.648278) (width 1) (layer B.Cu) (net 37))
 (segment (start 254.4 55.1) (end 253.6 55.9) (width 1) (layer B.Cu) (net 37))
 (segment (start 257.9 56.648278) (end 257.9 56.3) (width 1) (layer B.Cu) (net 37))
 (segment (start 262 86) (end 262.275 86) (width 1) (layer B.Cu) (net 37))
 (segment (start 257.9 56.3) (end 256.7 55.1) (width 1) (layer B.Cu) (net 37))
 (segment (start 251.56 84) (end 249.13 81.57) (width 1) (layer B.Cu) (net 36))
 (segment (start 262 84) (end 251.56 84) (width 1) (layer B.Cu) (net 36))
 (segment (start 262.275 84) (end 266.8 79.475) (width 1) (layer B.Cu) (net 36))
 (segment (start 262 84) (end 262.275 84) (width 1) (layer B.Cu) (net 36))
 (segment (start 266.8 67.9) (end 255.9 57) (width 1) (layer B.Cu) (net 36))
 (segment (start 266.8 79.475) (end 266.8 67.9) (width 1) (layer B.Cu) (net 36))
 (segment (start 255.9 64.62) (end 258 66.72) (width 1) (layer B.Cu) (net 33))
 (segment (start 258 66.72) (end 258 78.1) (width 1) (layer B.Cu) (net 33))
 (segment (start 258 78.1) (end 256.5 79.6) (width 1) (layer B.Cu) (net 33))
 (segment (start 254.78 79.6) (end 249.13 73.95) (width 1) (layer B.Cu) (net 33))
 (segment (start 256.5 79.6) (end 254.78 79.6) (width 1) (layer B.Cu) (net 33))
 (segment (start 246.9 59.02) (end 249.13 61.25) (width 1) (layer B.Cu) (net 28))
 (segment (start 246.9 40.8) (end 246.9 59.02) (width 1) (layer B.Cu) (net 28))
 (segment (start 251.3 40.8) (end 246.9 40.8) (width 1) (layer B.Cu) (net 28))
 (segment (start 252.39999 57.74292) (end 252.39999 41.89999) (width 1) (layer B.Cu) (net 28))
 (segment (start 254.200009 59.542939) (end 252.39999 57.74292) (width 1) (layer B.Cu) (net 28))
 (segment (start 252.39999 41.89999) (end 251.3 40.8) (width 1) (layer B.Cu) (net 28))
 (segment (start 255.011001 66.271001) (end 254.971001 66.271001) (width 1) (layer B.Cu) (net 28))
 (segment (start 255.9 67.16) (end 255.011001 66.271001) (width 1) (layer B.Cu) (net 28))
 (segment (start 254.971001 66.271001) (end 254.2 65.5) (width 1) (layer B.Cu) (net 28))
 (segment (start 254.2 65.5) (end 254.2 60.53707) (width 1) (layer B.Cu) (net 28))
 (segment (start 254.2 60.53707) (end 254.200009 60.537061) (width 1) (layer B.Cu) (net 28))
 (segment (start 254.200009 60.537061) (end 254.200009 59.542939) (width 1) (layer B.Cu) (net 28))
 (segment (start 255.8 69.7) (end 255.9 69.7) (width 1) (layer B.Cu) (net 26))
 (segment (start 255.5 69.4) (end 255.8 69.7) (width 1) (layer B.Cu) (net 26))
 (segment (start 254.9 69.4) (end 255.5 69.4) (width 1) (layer B.Cu) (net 26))
 (segment (start 252.7 67.2) (end 254.9 69.4) (width 1) (layer B.Cu) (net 26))
 (segment (start 252.7 59.74) (end 252.7 67.2) (width 1) (layer B.Cu) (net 26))
 (segment (start 249.13 56.17) (end 252.7 59.74) (width 1) (layer B.Cu) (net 26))
 (segment (start 255.9 72.24) (end 251.3 67.64) (width 1) (layer B.Cu) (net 27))
 (segment (start 251.3 67.64) (end 251.3 60.6) (width 1) (layer B.Cu) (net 27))
 (segment (start 251.02 60.6) (end 249.13 58.71) (width 1) (layer B.Cu) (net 27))
 (segment (start 251.3 60.6) (end 251.02 60.6) (width 1) (layer B.Cu) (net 27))
 (segment (start 255.04 74.78) (end 249.13 68.87) (width 1) (layer B.Cu) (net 31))
 (segment (start 255.9 74.78) (end 255.04 74.78) (width 1) (layer B.Cu) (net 31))
 (segment (start 255.04 77.32) (end 249.13 71.41) (width 1) (layer B.Cu) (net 32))
 (segment (start 255.9 77.32) (end 255.04 77.32) (width 1) (layer B.Cu) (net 32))
 (segment (start 255.72501 94.27499) (end 246.87499 94.27499) (width 1) (layer B.Cu) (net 35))
 (segment (start 262 88) (end 255.72501 94.27499) (width 1) (layer B.Cu) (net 35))
 (segment (start 246.87499 94.27499) (end 246.6 94) (width 1) (layer B.Cu) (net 35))
 (segment (start 246.6 81.56) (end 249.13 79.03) (width 1) (layer B.Cu) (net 35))
 (segment (start 246.6 94) (end 246.6 81.56) (width 1) (layer B.Cu) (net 35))
 (segment (start 221.6 89.75) (end 221.05 90.3) (width 1) (layer B.Cu) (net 47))
 (segment (start 221.6 88) (end 221.6 89.75) (width 1) (layer B.Cu) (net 47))
 (segment (start 212.9 87.6) (end 211.3 87.6) (width 1) (layer B.Cu) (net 47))
 (segment (start 215.6 90.3) (end 212.9 87.6) (width 1) (layer B.Cu) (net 47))
 (segment (start 221.05 90.3) (end 215.6 90.3) (width 1) (layer B.Cu) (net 47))
 (segment (start 211.42 82.9) (end 216.52 88) (width 1) (layer B.Cu) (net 49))
 (segment (start 207.2 82.9) (end 211.42 82.9) (width 1) (layer B.Cu) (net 49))
 (segment (start 212.75999 81.69999) (end 212.69999 81.69999) (width 1) (layer B.Cu) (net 48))
 (segment (start 219.06 88) (end 212.75999 81.69999) (width 1) (layer B.Cu) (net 48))
 (segment (start 212.69999 81.69999) (end 211.5 80.5) (width 1) (layer B.Cu) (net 48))
 (segment (start 211.5 80.5) (end 205.3 80.5) (width 1) (layer B.Cu) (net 48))
 (segment (start 205.3 80.5) (end 203.8 82) (width 1) (layer B.Cu) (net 48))
 (segment (start 197.49 90.3) (end 196.5 90.3) (width 1) (layer B.Cu) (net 48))
 (segment (start 203.8 83.99) (end 197.49 90.3) (width 1) (layer B.Cu) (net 48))
 (segment (start 203.8 82) (end 203.8 83.99) (width 1) (layer B.Cu) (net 48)))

